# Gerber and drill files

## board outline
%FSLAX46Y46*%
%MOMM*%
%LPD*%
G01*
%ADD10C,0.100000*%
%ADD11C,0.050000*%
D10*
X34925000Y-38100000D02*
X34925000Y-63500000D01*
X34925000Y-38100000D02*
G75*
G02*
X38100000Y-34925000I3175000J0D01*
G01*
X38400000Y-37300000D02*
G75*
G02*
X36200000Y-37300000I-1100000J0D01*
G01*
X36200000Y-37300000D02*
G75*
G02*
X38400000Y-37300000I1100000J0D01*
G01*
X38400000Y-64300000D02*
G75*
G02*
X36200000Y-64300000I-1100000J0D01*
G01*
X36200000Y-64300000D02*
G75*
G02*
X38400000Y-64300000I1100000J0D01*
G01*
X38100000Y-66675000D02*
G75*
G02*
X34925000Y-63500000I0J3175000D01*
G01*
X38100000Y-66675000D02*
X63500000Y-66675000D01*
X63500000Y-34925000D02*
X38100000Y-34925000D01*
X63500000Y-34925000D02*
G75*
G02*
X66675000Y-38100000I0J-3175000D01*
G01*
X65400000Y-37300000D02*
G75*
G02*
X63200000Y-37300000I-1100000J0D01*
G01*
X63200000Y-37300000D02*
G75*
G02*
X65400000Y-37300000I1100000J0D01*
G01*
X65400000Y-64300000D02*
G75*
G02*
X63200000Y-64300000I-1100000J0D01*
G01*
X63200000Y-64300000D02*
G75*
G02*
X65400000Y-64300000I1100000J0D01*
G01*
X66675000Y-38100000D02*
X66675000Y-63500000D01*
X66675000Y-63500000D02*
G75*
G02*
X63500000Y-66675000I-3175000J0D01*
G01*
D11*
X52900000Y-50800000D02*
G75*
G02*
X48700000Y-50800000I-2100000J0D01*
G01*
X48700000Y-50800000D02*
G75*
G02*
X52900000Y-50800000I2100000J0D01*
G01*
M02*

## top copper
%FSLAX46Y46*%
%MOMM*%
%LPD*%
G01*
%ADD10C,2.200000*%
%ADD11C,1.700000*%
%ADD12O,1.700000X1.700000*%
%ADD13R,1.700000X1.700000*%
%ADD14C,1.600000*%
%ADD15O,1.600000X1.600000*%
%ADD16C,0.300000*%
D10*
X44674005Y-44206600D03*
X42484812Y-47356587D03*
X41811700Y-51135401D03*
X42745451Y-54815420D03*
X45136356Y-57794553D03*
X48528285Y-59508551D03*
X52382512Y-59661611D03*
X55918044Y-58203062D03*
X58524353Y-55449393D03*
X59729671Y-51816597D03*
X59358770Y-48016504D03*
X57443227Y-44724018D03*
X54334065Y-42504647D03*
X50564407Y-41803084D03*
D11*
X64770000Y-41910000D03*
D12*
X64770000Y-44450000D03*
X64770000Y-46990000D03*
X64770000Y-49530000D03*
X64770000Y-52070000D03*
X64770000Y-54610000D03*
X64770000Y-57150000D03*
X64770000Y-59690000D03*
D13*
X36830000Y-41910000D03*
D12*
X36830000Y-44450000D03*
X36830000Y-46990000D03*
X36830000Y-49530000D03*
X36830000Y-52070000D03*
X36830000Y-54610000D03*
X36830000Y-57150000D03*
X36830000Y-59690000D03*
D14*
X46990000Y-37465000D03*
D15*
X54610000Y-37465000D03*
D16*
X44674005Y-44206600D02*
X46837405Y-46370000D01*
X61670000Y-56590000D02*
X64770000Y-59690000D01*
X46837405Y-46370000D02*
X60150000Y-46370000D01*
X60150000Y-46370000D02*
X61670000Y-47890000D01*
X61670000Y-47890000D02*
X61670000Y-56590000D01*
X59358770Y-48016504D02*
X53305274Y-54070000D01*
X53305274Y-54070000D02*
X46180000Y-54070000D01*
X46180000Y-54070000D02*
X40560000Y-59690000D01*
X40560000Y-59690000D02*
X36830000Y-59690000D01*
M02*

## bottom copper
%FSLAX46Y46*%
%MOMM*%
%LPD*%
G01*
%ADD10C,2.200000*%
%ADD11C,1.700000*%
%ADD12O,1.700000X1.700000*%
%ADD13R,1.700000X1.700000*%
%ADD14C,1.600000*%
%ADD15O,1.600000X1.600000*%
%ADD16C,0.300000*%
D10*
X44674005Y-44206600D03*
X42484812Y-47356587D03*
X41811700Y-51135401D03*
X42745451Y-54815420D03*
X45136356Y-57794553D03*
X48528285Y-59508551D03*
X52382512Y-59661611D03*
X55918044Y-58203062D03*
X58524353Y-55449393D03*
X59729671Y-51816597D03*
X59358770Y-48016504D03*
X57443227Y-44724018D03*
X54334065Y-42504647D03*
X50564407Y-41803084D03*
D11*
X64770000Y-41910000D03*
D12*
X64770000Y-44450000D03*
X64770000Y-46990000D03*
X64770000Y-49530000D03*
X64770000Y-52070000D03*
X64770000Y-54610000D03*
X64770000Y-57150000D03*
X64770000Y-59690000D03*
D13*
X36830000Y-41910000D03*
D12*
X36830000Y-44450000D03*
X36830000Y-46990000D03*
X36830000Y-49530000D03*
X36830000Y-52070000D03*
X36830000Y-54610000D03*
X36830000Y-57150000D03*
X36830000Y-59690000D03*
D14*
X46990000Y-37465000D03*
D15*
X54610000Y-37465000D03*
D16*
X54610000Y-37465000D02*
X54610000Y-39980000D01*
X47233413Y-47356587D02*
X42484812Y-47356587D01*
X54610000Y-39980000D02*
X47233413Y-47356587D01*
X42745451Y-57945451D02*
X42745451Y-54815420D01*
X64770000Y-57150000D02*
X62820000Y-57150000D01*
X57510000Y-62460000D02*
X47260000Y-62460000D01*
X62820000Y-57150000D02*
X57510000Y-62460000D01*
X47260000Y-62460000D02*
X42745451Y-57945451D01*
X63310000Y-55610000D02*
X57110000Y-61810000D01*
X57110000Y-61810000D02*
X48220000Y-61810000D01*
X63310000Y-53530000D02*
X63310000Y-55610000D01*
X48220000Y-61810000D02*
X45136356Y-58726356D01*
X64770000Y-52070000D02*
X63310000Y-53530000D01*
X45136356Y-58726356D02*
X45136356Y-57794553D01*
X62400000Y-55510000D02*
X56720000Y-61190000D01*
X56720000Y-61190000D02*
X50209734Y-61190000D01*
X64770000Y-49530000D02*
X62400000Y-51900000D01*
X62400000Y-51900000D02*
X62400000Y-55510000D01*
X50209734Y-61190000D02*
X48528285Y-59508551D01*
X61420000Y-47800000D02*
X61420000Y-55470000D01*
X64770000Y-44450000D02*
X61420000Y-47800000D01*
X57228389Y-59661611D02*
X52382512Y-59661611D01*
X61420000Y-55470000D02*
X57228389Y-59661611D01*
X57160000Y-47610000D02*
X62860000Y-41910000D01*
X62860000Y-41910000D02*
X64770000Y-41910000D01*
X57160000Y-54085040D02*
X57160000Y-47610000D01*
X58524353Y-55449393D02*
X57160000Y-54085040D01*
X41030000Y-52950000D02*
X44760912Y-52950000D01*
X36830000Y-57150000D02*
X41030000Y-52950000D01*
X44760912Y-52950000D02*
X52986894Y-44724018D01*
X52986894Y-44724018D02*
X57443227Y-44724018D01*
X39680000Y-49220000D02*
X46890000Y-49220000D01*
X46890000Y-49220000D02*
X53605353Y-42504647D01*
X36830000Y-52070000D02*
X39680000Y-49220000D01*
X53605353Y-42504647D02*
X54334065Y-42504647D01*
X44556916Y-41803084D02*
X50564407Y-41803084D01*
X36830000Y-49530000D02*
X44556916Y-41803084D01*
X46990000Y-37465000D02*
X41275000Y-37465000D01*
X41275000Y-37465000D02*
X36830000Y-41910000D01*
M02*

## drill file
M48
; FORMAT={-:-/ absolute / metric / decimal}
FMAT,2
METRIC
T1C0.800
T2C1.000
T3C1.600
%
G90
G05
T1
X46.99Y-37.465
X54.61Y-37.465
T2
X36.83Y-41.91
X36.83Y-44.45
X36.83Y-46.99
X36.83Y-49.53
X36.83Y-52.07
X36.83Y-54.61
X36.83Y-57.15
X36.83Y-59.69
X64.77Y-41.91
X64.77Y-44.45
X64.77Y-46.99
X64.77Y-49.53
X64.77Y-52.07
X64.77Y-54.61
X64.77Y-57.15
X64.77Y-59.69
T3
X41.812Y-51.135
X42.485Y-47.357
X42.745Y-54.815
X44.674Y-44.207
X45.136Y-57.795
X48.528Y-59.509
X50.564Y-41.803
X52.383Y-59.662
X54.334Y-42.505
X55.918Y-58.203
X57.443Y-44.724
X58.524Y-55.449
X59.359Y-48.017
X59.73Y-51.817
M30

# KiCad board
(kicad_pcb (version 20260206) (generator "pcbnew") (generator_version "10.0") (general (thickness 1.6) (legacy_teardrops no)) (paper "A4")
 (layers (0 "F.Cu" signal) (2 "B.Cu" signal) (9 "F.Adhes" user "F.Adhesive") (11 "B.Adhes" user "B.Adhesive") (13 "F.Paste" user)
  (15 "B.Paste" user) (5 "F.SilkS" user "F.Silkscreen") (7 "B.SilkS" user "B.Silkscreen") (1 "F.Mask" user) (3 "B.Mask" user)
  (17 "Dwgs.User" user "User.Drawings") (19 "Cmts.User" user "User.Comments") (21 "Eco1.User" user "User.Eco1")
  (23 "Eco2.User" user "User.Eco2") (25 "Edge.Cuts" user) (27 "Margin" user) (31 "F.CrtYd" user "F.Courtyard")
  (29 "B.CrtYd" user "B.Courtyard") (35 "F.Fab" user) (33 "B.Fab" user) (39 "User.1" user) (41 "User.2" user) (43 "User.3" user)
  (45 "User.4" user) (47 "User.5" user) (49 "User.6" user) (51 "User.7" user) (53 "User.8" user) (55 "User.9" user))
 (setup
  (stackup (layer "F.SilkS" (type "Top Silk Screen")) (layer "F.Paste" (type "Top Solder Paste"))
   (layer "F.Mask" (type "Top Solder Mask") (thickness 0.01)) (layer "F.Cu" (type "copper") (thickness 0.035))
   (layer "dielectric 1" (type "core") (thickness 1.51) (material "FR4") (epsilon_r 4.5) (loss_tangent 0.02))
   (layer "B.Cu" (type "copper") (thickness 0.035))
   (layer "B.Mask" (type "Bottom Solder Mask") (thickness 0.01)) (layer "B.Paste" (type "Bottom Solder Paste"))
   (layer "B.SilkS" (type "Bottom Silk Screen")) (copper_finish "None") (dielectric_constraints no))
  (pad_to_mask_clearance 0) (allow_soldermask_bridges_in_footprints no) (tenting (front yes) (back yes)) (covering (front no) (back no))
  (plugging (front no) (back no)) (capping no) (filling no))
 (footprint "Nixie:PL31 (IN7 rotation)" (layer "F.Cu") (at 50.8 50.8 180)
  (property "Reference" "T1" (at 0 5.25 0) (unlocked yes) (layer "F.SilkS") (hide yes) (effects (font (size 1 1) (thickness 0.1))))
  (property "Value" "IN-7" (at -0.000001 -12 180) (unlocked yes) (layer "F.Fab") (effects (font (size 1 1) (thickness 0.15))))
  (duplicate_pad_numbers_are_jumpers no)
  (fp_circle (center 0 0) (end 2.1 0) (stroke (width 0.05) (type default)) (fill no) (layer "Edge.Cuts"))
  (pad "1" thru_hole circle (at 6.125995 6.5934 1.5) (size 2.2 2.2) (drill 1.6) (layers "*.Cu" "*.Mask") (remove_unused_layers no)
   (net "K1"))
  (pad "2" thru_hole circle (at 8.315188 3.443413 1.5) (size 2.2 2.2) (drill 1.6) (layers "*.Cu" "*.Mask") (remove_unused_layers no)
   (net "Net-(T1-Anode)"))
  (pad "3" thru_hole circle (at 8.9883 -0.335401 1.5) (size 2.2 2.2) (drill 1.6) (layers "*.Cu" "*.Mask") (remove_unused_layers no)
   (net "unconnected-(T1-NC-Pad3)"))
  (pad "4" thru_hole circle (at 8.054549 -4.01542 1.5) (size 2.2 2.2) (drill 1.6) (layers "*.Cu" "*.Mask") (remove_unused_layers no)
   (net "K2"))
  (pad "5" thru_hole circle (at 5.663644 -6.994553 1.5) (size 2.2 2.2) (drill 1.6) (layers "*.Cu" "*.Mask") (remove_unused_layers no)
   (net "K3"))
  (pad "6" thru_hole circle (at 2.271715 -8.708551 1.5) (size 2.2 2.2) (drill 1.6) (layers "*.Cu" "*.Mask") (remove_unused_layers no)
   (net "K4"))
  (pad "7" thru_hole circle (at -1.582512 -8.861611 1.5) (size 2.2 2.2) (drill 1.6) (layers "*.Cu" "*.Mask") (remove_unused_layers no)
   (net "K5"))
  (pad "8" thru_hole circle (at -5.118044 -7.403062 1.5) (size 2.2 2.2) (drill 1.6) (layers "*.Cu" "*.Mask") (remove_unused_layers no)
   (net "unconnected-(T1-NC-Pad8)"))
  (pad "9" thru_hole circle (at -7.724353 -4.649393 1.5) (size 2.2 2.2) (drill 1.6) (layers "*.Cu" "*.Mask") (remove_unused_layers no)
   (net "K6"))
  (pad "10" thru_hole circle (at -8.929671 -1.016597 1.5) (size 2.2 2.2) (drill 1.6) (layers "*.Cu" "*.Mask") (remove_unused_layers no)
   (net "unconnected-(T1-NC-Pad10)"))
  (pad "11" thru_hole circle (at -8.55877 2.783496 1.5) (size 2.2 2.2) (drill 1.6) (layers "*.Cu" "*.Mask") (remove_unused_layers no)
   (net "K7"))
  (pad "12" thru_hole circle (at -6.643227 6.075982 1.5) (size 2.2 2.2) (drill 1.6) (layers "*.Cu" "*.Mask") (remove_unused_layers no)
   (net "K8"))
  (pad "13" thru_hole circle (at -3.534065 8.295353 1.5) (size 2.2 2.2) (drill 1.6) (layers "*.Cu" "*.Mask") (remove_unused_layers no)
   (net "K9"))
  (pad "14" thru_hole circle (at 0.235593 8.996916 1.5) (size 2.2 2.2) (drill 1.6) (layers "*.Cu" "*.Mask") (remove_unused_layers no)
   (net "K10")))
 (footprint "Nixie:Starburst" (layer "F.Cu") (at 43 63.25)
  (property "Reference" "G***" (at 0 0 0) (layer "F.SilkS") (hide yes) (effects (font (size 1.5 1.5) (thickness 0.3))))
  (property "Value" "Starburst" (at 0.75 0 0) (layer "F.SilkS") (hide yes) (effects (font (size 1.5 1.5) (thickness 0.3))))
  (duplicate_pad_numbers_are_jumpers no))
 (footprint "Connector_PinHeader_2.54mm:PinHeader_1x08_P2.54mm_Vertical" (layer "B.Cu") (at 64.77 41.91 180)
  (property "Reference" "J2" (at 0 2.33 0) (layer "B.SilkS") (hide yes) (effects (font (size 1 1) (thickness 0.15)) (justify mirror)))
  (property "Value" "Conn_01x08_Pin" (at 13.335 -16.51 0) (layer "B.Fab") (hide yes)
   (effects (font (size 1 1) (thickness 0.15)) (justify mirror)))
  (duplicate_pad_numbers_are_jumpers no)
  (pad "1" thru_hole circle (at 0 0 180) (size 1.7 1.7) (drill 1) (layers "*.Cu" "*.Mask") (remove_unused_layers no) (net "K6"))
  (pad "2" thru_hole oval (at 0 -2.54 180) (size 1.7 1.7) (drill 1) (layers "*.Cu" "*.Mask") (remove_unused_layers no) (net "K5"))
  (pad "3" thru_hole oval (at 0 -5.08 180) (size 1.7 1.7) (drill 1) (layers "*.Cu" "*.Mask") (remove_unused_layers no)
   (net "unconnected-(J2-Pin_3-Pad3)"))
  (pad "4" thru_hole oval (at 0 -7.62 180) (size 1.7 1.7) (drill 1) (layers "*.Cu" "*.Mask") (remove_unused_layers no) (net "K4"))
  (pad "5" thru_hole oval (at 0 -10.16 180) (size 1.7 1.7) (drill 1) (layers "*.Cu" "*.Mask") (remove_unused_layers no) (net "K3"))
  (pad "6" thru_hole oval (at 0 -12.7 180) (size 1.7 1.7) (drill 1) (layers "*.Cu" "*.Mask") (remove_unused_layers no)
   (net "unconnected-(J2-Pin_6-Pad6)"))
  (pad "7" thru_hole oval (at 0 -15.24 180) (size 1.7 1.7) (drill 1) (layers "*.Cu" "*.Mask") (remove_unused_layers no) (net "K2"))
  (pad "8" thru_hole oval (at 0 -17.78 180) (size 1.7 1.7) (drill 1) (layers "*.Cu" "*.Mask") (remove_unused_layers no) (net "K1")))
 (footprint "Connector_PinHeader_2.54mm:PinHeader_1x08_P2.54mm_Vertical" (layer "B.Cu") (at 36.83 41.91 180)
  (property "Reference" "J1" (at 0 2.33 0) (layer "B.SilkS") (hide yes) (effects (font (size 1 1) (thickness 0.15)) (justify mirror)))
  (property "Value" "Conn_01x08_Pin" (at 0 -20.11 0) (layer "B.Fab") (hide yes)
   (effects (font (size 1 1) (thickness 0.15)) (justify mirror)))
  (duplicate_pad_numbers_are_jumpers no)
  (pad "1" thru_hole rect (at 0 0 180) (size 1.7 1.7) (drill 1) (layers "*.Cu" "*.Mask") (remove_unused_layers no) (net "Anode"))
  (pad "2" thru_hole oval (at 0 -2.54 180) (size 1.7 1.7) (drill 1) (layers "*.Cu" "*.Mask") (remove_unused_layers no)
   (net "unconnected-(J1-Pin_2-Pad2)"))
  (pad "3" thru_hole oval (at 0 -5.08 180) (size 1.7 1.7) (drill 1) (layers "*.Cu" "*.Mask") (remove_unused_layers no)
   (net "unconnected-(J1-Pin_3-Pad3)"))
  (pad "4" thru_hole oval (at 0 -7.62 180) (size 1.7 1.7) (drill 1) (layers "*.Cu" "*.Mask") (remove_unused_layers no) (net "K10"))
  (pad "5" thru_hole oval (at 0 -10.16 180) (size 1.7 1.7) (drill 1) (layers "*.Cu" "*.Mask") (remove_unused_layers no) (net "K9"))
  (pad "6" thru_hole oval (at 0 -12.7 180) (size 1.7 1.7) (drill 1) (layers "*.Cu" "*.Mask") (remove_unused_layers no)
   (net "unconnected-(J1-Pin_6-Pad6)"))
  (pad "7" thru_hole oval (at 0 -15.24 180) (size 1.7 1.7) (drill 1) (layers "*.Cu" "*.Mask") (remove_unused_layers no) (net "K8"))
  (pad "8" thru_hole oval (at 0 -17.78 180) (size 1.7 1.7) (drill 1) (layers "*.Cu" "*.Mask") (remove_unused_layers no) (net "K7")))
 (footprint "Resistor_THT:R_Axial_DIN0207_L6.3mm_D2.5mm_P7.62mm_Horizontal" (layer "B.Cu") (at 46.99 37.465)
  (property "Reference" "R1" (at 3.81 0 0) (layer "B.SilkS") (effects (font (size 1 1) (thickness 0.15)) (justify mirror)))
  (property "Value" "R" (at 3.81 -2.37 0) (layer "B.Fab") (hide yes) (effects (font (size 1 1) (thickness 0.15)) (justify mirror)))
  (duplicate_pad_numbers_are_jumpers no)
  (pad "1" thru_hole circle (at 0 0) (size 1.6 1.6) (drill 0.8) (layers "*.Cu" "*.Mask") (remove_unused_layers no) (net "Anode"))
  (pad "2" thru_hole oval (at 7.62 0) (size 1.6 1.6) (drill 0.8) (layers "*.Cu" "*.Mask") (remove_unused_layers no) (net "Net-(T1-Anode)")))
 (gr_line (start 34.925 38.1) (end 34.925 63.5) (stroke (width 0.1) (type default)) (layer "Edge.Cuts"))
 (gr_arc (start 34.925 38.1) (mid 35.854936 35.854936) (end 38.1 34.925) (stroke (width 0.1) (type default)) (layer "Edge.Cuts"))
 (gr_circle (center 37.3 37.3) (end 38.4 37.3) (stroke (width 0.1) (type default)) (fill no) (layer "Edge.Cuts"))
 (gr_circle (center 37.3 64.3) (end 38.4 64.3) (stroke (width 0.1) (type default)) (fill no) (layer "Edge.Cuts"))
 (gr_arc (start 38.1 66.675) (mid 35.854936 65.745064) (end 34.925 63.5) (stroke (width 0.1) (type default)) (layer "Edge.Cuts"))
 (gr_line (start 38.1 66.675) (end 63.5 66.675) (stroke (width 0.1) (type default)) (layer "Edge.Cuts"))
 (gr_line (start 63.5 34.925) (end 38.1 34.925) (stroke (width 0.1) (type default)) (layer "Edge.Cuts"))
 (gr_arc (start 63.5 34.925) (mid 65.745064 35.854936) (end 66.675 38.1) (stroke (width 0.1) (type default)) (layer "Edge.Cuts"))
 (gr_circle (center 64.3 37.3) (end 65.4 37.3) (stroke (width 0.1) (type default)) (fill no) (layer "Edge.Cuts"))
 (gr_circle (center 64.3 64.3) (end 65.4 64.3) (stroke (width 0.1) (type default)) (fill no) (layer "Edge.Cuts"))
 (gr_line (start 66.675 38.1) (end 66.675 63.5) (stroke (width 0.1) (type default)) (layer "Edge.Cuts"))
 (gr_arc (start 66.675 63.5) (mid 65.745064 65.745064) (end 63.5 66.675) (stroke (width 0.1) (type default)) (layer "Edge.Cuts"))
 (segment (start 44.674005 44.2066) (end 46.837405 46.37) (width 0.3) (layer "F.Cu") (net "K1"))
 (segment (start 61.67 56.59) (end 64.77 59.69) (width 0.3) (layer "F.Cu") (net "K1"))
 (segment (start 46.837405 46.37) (end 60.15 46.37) (width 0.3) (layer "F.Cu") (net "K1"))
 (segment (start 60.15 46.37) (end 61.67 47.89) (width 0.3) (layer "F.Cu") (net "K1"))
 (segment (start 61.67 47.89) (end 61.67 56.59) (width 0.3) (layer "F.Cu") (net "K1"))
 (segment (start 54.61 37.465) (end 54.61 39.98) (width 0.3) (layer "B.Cu") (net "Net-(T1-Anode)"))
 (segment (start 47.233413 47.356587) (end 42.484812 47.356587) (width 0.3) (layer "B.Cu") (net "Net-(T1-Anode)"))
 (segment (start 54.61 39.98) (end 47.233413 47.356587) (width 0.3) (layer "B.Cu") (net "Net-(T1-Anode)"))
 (segment (start 42.745451 57.945451) (end 42.745451 54.81542) (width 0.3) (layer "B.Cu") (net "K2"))
 (segment (start 64.77 57.15) (end 62.82 57.15) (width 0.3) (layer "B.Cu") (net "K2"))
 (segment (start 57.51 62.46) (end 47.26 62.46) (width 0.3) (layer "B.Cu") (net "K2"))
 (segment (start 62.82 57.15) (end 57.51 62.46) (width 0.3) (layer "B.Cu") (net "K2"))
 (segment (start 47.26 62.46) (end 42.745451 57.945451) (width 0.3) (layer "B.Cu") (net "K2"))
 (segment (start 63.31 55.61) (end 57.11 61.81) (width 0.3) (layer "B.Cu") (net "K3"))
 (segment (start 57.11 61.81) (end 48.22 61.81) (width 0.3) (layer "B.Cu") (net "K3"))
 (segment (start 63.31 53.53) (end 63.31 55.61) (width 0.3) (layer "B.Cu") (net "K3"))
 (segment (start 48.22 61.81) (end 45.136356 58.726356) (width 0.3) (layer "B.Cu") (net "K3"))
 (segment (start 64.77 52.07) (end 63.31 53.53) (width 0.3) (layer "B.Cu") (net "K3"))
 (segment (start 45.136356 58.726356) (end 45.136356 57.794553) (width 0.3) (layer "B.Cu") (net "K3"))
 (segment (start 62.4 55.51) (end 56.72 61.19) (width 0.3) (layer "B.Cu") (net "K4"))
 (segment (start 56.72 61.19) (end 50.209734 61.19) (width 0.3) (layer "B.Cu") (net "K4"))
 (segment (start 64.77 49.53) (end 62.4 51.9) (width 0.3) (layer "B.Cu") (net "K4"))
 (segment (start 62.4 51.9) (end 62.4 55.51) (width 0.3) (layer "B.Cu") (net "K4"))
 (segment (start 50.209734 61.19) (end 48.528285 59.508551) (width 0.3) (layer "B.Cu") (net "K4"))
 (segment (start 61.42 47.8) (end 61.42 55.47) (width 0.3) (layer "B.Cu") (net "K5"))
 (segment (start 64.77 44.45) (end 61.42 47.8) (width 0.3) (layer "B.Cu") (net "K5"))
 (segment (start 57.228389 59.661611) (end 52.382512 59.661611) (width 0.3) (layer "B.Cu") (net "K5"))
 (segment (start 61.42 55.47) (end 57.228389 59.661611) (width 0.3) (layer "B.Cu") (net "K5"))
 (segment (start 57.16 47.61) (end 62.86 41.91) (width 0.3) (layer "B.Cu") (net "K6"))
 (segment (start 62.86 41.91) (end 64.77 41.91) (width 0.3) (layer "B.Cu") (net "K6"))
 (segment (start 57.16 54.08504) (end 57.16 47.61) (width 0.3) (layer "B.Cu") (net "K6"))
 (segment (start 58.524353 55.449393) (end 57.16 54.08504) (width 0.3) (layer "B.Cu") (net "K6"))
 (segment (start 59.35877 48.016504) (end 53.305274 54.07) (width 0.3) (layer "F.Cu") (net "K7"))
 (segment (start 53.305274 54.07) (end 46.18 54.07) (width 0.3) (layer "F.Cu") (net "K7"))
 (segment (start 46.18 54.07) (end 40.56 59.69) (width 0.3) (layer "F.Cu") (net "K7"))
 (segment (start 40.56 59.69) (end 36.83 59.69) (width 0.3) (layer "F.Cu") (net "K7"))
 (segment (start 41.03 52.95) (end 44.760912 52.95) (width 0.3) (layer "B.Cu") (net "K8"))
 (segment (start 36.83 57.15) (end 41.03 52.95) (width 0.3) (layer "B.Cu") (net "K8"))
 (segment (start 44.760912 52.95) (end 52.986894 44.724018) (width 0.3) (layer "B.Cu") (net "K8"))
 (segment (start 52.986894 44.724018) (end 57.443227 44.724018) (width 0.3) (layer "B.Cu") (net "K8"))
 (segment (start 39.68 49.22) (end 46.89 49.22) (width 0.3) (layer "B.Cu") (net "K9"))
 (segment (start 46.89 49.22) (end 53.605353 42.504647) (width 0.3) (layer "B.Cu") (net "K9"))
 (segment (start 36.83 52.07) (end 39.68 49.22) (width 0.3) (layer "B.Cu") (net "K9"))
 (segment (start 53.605353 42.504647) (end 54.334065 42.504647) (width 0.3) (layer "B.Cu") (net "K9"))
 (segment (start 44.556916 41.803084) (end 50.564407 41.803084) (width 0.3) (layer "B.Cu") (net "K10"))
 (segment (start 36.83 49.53) (end 44.556916 41.803084) (width 0.3) (layer "B.Cu") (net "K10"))
 (segment (start 46.99 37.465) (end 41.275 37.465) (width 0.3) (layer "B.Cu") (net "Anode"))
 (segment (start 41.275 37.465) (end 36.83 41.91) (width 0.3) (layer "B.Cu") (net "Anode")))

